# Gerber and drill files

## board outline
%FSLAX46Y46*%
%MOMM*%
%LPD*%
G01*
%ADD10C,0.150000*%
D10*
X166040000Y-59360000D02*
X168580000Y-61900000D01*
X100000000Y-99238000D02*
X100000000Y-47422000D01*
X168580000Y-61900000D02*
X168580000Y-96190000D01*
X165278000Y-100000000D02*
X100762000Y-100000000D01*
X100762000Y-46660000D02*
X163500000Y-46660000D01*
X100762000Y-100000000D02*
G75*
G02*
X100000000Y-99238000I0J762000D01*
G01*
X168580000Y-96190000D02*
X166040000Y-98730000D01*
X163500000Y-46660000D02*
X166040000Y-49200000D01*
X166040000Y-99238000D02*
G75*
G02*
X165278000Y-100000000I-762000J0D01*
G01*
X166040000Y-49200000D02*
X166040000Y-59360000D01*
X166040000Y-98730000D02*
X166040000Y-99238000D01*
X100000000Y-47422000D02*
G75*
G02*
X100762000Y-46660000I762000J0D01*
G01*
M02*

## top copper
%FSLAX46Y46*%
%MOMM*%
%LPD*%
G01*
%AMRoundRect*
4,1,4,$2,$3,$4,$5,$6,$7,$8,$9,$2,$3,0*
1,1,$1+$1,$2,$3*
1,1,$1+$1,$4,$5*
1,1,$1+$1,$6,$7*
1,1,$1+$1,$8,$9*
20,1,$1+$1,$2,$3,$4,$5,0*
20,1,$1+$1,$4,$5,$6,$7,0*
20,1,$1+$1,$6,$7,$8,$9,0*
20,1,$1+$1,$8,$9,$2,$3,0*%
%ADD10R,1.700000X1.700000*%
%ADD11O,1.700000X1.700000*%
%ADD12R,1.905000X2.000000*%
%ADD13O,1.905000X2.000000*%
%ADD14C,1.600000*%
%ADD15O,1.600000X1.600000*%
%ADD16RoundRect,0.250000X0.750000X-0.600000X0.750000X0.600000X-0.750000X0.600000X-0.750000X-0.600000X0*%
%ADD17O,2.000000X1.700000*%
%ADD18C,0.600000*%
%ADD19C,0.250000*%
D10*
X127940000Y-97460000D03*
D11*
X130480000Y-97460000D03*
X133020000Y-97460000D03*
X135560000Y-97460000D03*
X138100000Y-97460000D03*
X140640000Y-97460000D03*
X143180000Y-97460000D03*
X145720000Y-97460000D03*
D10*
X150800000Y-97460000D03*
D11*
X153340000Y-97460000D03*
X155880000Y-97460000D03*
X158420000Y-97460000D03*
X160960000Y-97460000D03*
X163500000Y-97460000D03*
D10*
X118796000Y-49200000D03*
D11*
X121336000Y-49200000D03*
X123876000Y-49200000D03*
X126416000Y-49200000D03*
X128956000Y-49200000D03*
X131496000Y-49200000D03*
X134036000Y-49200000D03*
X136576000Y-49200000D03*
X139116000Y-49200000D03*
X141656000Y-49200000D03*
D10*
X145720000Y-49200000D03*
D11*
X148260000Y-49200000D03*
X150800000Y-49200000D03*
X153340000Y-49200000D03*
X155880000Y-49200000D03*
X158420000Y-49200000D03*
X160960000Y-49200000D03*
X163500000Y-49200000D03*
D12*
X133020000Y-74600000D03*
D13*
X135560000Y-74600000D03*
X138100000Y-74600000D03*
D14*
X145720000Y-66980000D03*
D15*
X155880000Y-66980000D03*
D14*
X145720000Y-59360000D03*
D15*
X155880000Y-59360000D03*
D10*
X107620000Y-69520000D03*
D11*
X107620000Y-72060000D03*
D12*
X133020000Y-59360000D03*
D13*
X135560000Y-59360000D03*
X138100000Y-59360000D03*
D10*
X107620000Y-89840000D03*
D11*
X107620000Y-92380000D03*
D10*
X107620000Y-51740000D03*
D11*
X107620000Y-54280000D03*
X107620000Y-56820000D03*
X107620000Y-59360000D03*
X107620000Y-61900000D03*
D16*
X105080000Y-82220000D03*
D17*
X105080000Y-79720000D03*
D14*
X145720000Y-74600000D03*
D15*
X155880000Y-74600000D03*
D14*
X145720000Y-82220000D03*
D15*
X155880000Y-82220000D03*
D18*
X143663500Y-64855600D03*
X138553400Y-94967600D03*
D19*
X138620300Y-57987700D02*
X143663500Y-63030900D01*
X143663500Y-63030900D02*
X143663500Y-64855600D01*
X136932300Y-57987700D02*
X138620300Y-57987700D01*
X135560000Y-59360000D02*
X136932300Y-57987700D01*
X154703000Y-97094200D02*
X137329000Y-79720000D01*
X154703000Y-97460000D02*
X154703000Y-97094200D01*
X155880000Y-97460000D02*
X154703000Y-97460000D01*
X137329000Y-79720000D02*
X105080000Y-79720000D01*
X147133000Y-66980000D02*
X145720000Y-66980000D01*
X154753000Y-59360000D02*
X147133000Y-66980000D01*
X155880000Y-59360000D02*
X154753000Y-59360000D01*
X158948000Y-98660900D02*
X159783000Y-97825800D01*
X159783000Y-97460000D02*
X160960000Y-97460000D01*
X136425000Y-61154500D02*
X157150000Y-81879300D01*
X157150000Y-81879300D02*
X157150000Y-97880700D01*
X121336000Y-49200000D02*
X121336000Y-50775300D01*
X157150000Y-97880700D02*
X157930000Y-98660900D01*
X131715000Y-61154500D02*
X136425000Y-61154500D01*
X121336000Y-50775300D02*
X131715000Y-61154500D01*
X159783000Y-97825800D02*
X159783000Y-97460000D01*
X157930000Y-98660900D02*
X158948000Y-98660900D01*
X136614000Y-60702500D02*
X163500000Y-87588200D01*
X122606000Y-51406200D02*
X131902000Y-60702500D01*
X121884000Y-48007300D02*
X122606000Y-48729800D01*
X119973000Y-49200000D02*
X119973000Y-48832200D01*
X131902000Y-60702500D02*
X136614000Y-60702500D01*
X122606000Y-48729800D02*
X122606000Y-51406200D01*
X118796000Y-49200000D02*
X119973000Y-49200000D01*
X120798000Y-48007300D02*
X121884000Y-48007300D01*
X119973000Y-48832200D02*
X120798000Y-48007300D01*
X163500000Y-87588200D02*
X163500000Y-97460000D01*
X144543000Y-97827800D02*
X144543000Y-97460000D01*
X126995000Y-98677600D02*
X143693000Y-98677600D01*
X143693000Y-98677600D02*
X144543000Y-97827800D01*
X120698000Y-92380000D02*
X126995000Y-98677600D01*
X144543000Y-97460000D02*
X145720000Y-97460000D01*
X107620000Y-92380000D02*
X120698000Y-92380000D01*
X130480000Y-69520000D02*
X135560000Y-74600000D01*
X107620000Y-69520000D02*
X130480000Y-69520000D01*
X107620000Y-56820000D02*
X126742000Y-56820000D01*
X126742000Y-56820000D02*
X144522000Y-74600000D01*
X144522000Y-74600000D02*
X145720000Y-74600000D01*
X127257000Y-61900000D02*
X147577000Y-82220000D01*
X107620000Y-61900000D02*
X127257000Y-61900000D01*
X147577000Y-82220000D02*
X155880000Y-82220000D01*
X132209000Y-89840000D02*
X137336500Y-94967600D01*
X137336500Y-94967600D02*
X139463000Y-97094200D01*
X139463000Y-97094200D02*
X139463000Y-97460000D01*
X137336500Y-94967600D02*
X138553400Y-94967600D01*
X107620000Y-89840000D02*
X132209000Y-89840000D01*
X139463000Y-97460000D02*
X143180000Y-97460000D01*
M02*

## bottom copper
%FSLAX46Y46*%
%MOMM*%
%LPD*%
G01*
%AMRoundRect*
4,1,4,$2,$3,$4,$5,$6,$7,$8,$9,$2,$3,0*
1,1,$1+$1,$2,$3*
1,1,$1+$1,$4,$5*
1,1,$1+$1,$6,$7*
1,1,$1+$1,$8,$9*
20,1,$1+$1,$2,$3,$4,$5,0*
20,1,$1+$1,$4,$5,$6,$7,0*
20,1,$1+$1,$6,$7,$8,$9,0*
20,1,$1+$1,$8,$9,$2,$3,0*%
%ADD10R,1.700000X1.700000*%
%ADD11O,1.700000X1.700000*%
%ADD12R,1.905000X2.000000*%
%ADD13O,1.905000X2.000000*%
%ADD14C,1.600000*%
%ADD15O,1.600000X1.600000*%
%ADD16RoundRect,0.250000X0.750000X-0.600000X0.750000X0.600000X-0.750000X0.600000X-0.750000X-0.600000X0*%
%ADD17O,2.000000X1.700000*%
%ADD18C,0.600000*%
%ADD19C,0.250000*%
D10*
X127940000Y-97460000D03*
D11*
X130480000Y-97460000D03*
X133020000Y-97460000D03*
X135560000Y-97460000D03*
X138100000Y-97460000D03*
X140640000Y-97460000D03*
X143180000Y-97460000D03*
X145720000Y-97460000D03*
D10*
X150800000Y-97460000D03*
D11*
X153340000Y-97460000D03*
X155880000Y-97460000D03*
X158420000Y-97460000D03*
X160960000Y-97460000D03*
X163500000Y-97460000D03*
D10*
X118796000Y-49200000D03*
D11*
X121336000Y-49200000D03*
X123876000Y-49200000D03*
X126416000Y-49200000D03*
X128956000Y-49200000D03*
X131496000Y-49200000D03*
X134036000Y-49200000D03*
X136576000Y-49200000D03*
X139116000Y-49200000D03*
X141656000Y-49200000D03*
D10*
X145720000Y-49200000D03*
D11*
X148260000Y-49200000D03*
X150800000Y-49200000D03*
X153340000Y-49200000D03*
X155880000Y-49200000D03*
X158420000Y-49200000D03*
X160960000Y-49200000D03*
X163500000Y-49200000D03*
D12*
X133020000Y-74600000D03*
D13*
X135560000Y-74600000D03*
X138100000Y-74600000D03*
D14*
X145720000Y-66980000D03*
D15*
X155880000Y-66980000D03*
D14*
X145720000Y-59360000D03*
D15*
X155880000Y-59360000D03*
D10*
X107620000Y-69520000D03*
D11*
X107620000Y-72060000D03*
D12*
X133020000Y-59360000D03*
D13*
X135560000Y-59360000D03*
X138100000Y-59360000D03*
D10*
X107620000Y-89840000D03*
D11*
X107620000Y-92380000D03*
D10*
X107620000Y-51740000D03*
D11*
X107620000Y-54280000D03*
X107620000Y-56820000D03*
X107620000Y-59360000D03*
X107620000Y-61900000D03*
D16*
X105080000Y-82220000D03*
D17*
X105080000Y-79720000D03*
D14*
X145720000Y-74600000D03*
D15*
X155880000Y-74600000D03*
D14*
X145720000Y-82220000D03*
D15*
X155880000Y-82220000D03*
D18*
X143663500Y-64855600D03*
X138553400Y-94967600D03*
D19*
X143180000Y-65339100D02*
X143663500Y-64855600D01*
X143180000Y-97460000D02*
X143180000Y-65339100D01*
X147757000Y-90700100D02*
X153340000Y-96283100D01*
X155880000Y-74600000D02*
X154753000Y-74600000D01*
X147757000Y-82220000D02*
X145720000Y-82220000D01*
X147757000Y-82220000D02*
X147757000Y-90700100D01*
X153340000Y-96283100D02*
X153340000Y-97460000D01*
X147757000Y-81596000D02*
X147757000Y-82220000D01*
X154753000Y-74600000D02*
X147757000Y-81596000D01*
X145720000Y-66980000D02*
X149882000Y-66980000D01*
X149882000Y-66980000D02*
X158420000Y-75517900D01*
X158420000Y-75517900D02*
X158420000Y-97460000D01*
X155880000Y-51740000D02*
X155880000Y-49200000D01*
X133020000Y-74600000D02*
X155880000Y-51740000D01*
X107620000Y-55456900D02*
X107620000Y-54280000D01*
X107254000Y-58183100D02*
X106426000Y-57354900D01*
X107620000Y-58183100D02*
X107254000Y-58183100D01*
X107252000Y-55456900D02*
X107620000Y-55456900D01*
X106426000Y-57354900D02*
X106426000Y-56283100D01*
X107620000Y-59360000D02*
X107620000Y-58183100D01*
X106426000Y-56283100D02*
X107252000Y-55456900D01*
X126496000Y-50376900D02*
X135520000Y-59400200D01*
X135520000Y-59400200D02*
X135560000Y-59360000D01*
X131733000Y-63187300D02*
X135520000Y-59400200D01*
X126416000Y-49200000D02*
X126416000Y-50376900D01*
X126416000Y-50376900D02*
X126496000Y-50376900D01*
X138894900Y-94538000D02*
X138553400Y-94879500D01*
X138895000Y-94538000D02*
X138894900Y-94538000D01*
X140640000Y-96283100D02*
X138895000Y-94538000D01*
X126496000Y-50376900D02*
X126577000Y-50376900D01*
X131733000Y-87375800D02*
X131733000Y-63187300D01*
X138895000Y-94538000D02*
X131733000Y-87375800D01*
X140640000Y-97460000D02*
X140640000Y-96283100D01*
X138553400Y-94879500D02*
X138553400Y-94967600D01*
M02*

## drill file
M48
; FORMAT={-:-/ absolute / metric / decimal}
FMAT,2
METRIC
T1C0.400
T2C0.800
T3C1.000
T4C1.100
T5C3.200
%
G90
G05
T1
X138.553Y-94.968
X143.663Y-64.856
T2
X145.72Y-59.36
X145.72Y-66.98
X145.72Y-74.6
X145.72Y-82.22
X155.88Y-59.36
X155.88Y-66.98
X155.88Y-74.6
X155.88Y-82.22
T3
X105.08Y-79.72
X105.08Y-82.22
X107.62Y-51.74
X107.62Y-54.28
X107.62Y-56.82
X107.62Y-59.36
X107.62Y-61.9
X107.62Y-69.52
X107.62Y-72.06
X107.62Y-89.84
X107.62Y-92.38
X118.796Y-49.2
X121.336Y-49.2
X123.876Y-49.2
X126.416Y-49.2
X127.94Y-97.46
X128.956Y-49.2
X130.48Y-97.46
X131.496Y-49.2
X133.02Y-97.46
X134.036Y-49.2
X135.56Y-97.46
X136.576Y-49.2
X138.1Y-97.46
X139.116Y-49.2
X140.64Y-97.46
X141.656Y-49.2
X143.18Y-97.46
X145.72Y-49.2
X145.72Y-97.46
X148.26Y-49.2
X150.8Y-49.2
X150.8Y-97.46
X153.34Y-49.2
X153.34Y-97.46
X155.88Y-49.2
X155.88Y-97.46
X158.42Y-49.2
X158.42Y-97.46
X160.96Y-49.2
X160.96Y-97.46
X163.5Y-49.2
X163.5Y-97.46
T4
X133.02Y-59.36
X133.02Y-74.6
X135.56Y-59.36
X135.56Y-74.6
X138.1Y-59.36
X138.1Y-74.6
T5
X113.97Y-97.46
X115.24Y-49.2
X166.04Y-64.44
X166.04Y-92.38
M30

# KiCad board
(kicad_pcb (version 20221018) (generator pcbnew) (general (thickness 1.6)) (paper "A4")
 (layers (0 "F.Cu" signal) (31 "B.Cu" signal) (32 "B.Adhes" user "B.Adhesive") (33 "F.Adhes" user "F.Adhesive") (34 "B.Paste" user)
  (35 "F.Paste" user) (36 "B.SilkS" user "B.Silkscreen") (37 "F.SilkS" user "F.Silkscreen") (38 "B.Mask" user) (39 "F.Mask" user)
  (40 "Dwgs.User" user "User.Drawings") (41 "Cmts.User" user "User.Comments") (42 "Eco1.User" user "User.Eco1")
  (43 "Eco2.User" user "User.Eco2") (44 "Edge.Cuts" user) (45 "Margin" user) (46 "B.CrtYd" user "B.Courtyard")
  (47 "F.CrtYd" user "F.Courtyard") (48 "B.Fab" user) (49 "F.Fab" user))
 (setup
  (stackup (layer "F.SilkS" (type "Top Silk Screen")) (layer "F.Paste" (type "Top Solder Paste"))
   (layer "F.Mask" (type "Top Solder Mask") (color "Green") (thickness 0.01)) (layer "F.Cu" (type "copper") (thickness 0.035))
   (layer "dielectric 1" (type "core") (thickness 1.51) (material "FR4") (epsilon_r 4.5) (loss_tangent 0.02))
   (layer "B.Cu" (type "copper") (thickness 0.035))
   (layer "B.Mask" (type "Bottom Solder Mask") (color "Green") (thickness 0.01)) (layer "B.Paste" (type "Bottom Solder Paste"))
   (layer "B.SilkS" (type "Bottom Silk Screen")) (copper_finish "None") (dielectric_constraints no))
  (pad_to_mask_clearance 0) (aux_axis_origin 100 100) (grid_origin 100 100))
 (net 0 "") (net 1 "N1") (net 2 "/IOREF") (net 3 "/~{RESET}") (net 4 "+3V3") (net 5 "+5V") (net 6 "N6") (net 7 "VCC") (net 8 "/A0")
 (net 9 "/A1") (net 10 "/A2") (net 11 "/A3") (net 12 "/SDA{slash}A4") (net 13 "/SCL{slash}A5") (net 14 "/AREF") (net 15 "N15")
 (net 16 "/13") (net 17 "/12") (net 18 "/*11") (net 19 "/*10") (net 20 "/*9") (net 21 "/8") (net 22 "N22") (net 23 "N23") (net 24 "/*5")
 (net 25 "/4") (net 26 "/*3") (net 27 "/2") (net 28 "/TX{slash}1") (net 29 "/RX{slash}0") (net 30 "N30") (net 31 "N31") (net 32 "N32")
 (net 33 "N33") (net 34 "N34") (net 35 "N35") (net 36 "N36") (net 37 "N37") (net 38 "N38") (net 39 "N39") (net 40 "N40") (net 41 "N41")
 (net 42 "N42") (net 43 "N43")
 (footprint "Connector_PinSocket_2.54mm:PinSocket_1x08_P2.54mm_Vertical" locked (layer "F.Cu") (at 127.94 97.46 90)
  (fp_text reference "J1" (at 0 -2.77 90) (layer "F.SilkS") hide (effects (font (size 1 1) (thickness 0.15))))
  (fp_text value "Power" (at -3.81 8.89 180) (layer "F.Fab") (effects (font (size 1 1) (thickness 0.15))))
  (pad "1" thru_hole rect locked (at 0 0 90) (size 1.7 1.7) (drill 1) (layers "*.Cu" "*.Mask") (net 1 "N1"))
  (pad "2" thru_hole oval locked (at 0 2.54 90) (size 1.7 1.7) (drill 1) (layers "*.Cu" "*.Mask") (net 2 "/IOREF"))
  (pad "3" thru_hole oval locked (at 0 5.08 90) (size 1.7 1.7) (drill 1) (layers "*.Cu" "*.Mask") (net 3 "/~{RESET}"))
  (pad "4" thru_hole oval locked (at 0 7.62 90) (size 1.7 1.7) (drill 1) (layers "*.Cu" "*.Mask") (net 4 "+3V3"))
  (pad "5" thru_hole oval locked (at 0 10.16 90) (size 1.7 1.7) (drill 1) (layers "*.Cu" "*.Mask") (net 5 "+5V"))
  (pad "6" thru_hole oval locked (at 0 12.7 90) (size 1.7 1.7) (drill 1) (layers "*.Cu" "*.Mask") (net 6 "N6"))
  (pad "7" thru_hole oval locked (at 0 15.24 90) (size 1.7 1.7) (drill 1) (layers "*.Cu" "*.Mask") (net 6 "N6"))
  (pad "8" thru_hole oval locked (at 0 17.78 90) (size 1.7 1.7) (drill 1) (layers "*.Cu" "*.Mask") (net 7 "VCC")))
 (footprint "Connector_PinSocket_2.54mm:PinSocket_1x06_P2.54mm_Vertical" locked (layer "F.Cu") (at 150.8 97.46 90)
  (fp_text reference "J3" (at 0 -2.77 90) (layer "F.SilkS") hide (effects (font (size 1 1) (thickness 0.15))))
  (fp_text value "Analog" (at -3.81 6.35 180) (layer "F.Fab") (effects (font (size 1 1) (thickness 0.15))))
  (pad "1" thru_hole rect locked (at 0 0 90) (size 1.7 1.7) (drill 1) (layers "*.Cu" "*.Mask") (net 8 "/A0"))
  (pad "2" thru_hole oval locked (at 0 2.54 90) (size 1.7 1.7) (drill 1) (layers "*.Cu" "*.Mask") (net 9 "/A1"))
  (pad "3" thru_hole oval locked (at 0 5.08 90) (size 1.7 1.7) (drill 1) (layers "*.Cu" "*.Mask") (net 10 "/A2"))
  (pad "4" thru_hole oval locked (at 0 7.62 90) (size 1.7 1.7) (drill 1) (layers "*.Cu" "*.Mask") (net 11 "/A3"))
  (pad "5" thru_hole oval locked (at 0 10.16 90) (size 1.7 1.7) (drill 1) (layers "*.Cu" "*.Mask") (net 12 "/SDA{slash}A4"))
  (pad "6" thru_hole oval locked (at 0 12.7 90) (size 1.7 1.7) (drill 1) (layers "*.Cu" "*.Mask") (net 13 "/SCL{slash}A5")))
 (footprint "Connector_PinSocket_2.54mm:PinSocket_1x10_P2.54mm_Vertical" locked (layer "F.Cu") (at 118.796 49.2 90)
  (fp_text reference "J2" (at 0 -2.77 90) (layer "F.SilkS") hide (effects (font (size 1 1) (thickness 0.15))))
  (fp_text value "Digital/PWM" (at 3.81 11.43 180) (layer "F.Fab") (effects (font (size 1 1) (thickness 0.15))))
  (pad "1" thru_hole rect locked (at 0 0 90) (size 1.7 1.7) (drill 1) (layers "*.Cu" "*.Mask") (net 13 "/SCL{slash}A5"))
  (pad "2" thru_hole oval locked (at 0 2.54 90) (size 1.7 1.7) (drill 1) (layers "*.Cu" "*.Mask") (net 12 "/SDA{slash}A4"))
  (pad "3" thru_hole oval locked (at 0 5.08 90) (size 1.7 1.7) (drill 1) (layers "*.Cu" "*.Mask") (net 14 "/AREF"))
  (pad "4" thru_hole oval locked (at 0 7.62 90) (size 1.7 1.7) (drill 1) (layers "*.Cu" "*.Mask") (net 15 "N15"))
  (pad "5" thru_hole oval locked (at 0 10.16 90) (size 1.7 1.7) (drill 1) (layers "*.Cu" "*.Mask") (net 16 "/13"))
  (pad "6" thru_hole oval locked (at 0 12.7 90) (size 1.7 1.7) (drill 1) (layers "*.Cu" "*.Mask") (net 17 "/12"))
  (pad "7" thru_hole oval locked (at 0 15.24 90) (size 1.7 1.7) (drill 1) (layers "*.Cu" "*.Mask") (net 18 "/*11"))
  (pad "8" thru_hole oval locked (at 0 17.78 90) (size 1.7 1.7) (drill 1) (layers "*.Cu" "*.Mask") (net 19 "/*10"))
  (pad "9" thru_hole oval locked (at 0 20.32 90) (size 1.7 1.7) (drill 1) (layers "*.Cu" "*.Mask") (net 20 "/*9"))
  (pad "10" thru_hole oval locked (at 0 22.86 90) (size 1.7 1.7) (drill 1) (layers "*.Cu" "*.Mask") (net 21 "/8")))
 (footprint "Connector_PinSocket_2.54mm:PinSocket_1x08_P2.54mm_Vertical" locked (layer "F.Cu") (at 145.72 49.2 90)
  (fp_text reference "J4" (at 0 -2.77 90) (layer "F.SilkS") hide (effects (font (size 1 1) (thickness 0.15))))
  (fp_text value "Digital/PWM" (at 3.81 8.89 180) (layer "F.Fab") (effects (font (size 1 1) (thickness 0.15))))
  (pad "1" thru_hole rect locked (at 0 0 90) (size 1.7 1.7) (drill 1) (layers "*.Cu" "*.Mask") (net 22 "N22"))
  (pad "2" thru_hole oval locked (at 0 2.54 90) (size 1.7 1.7) (drill 1) (layers "*.Cu" "*.Mask") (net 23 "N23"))
  (pad "3" thru_hole oval locked (at 0 5.08 90) (size 1.7 1.7) (drill 1) (layers "*.Cu" "*.Mask") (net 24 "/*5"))
  (pad "4" thru_hole oval locked (at 0 7.62 90) (size 1.7 1.7) (drill 1) (layers "*.Cu" "*.Mask") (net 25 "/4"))
  (pad "5" thru_hole oval locked (at 0 10.16 90) (size 1.7 1.7) (drill 1) (layers "*.Cu" "*.Mask") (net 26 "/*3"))
  (pad "6" thru_hole oval locked (at 0 12.7 90) (size 1.7 1.7) (drill 1) (layers "*.Cu" "*.Mask") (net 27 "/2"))
  (pad "7" thru_hole oval locked (at 0 15.24 90) (size 1.7 1.7) (drill 1) (layers "*.Cu" "*.Mask") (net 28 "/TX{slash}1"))
  (pad "8" thru_hole oval locked (at 0 17.78 90) (size 1.7 1.7) (drill 1) (layers "*.Cu" "*.Mask") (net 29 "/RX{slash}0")))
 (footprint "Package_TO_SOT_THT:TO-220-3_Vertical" (layer "F.Cu") (at 133.02 74.6)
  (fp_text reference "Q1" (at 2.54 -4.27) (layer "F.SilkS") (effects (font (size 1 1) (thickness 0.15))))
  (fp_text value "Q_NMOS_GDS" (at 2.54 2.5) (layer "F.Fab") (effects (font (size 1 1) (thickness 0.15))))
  (pad "1" thru_hole rect (at 0 0) (size 1.905 2) (drill 1.1) (layers "*.Cu" "*.Mask") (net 26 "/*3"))
  (pad "2" thru_hole oval (at 2.54 0) (size 1.905 2) (drill 1.1) (layers "*.Cu" "*.Mask") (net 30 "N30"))
  (pad "3" thru_hole oval (at 5.08 0) (size 1.905 2) (drill 1.1) (layers "*.Cu" "*.Mask") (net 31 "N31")))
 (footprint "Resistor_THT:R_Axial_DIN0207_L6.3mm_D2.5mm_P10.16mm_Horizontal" (layer "F.Cu") (at 145.72 66.98)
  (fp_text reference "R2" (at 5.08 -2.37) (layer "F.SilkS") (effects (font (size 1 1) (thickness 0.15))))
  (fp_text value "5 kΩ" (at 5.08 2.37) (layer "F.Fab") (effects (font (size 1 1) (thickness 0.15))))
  (pad "1" thru_hole circle (at 0 0) (size 1.6 1.6) (drill 0.8) (layers "*.Cu" "*.Mask") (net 11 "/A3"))
  (pad "2" thru_hole oval (at 10.16 0) (size 1.6 1.6) (drill 0.8) (layers "*.Cu" "*.Mask") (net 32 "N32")))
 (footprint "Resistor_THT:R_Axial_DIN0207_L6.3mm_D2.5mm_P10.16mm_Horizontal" (layer "F.Cu") (at 145.72 59.36)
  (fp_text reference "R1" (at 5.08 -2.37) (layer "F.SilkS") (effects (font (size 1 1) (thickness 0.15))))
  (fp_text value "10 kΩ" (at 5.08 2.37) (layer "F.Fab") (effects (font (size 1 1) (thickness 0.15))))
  (pad "1" thru_hole circle (at 0 0) (size 1.6 1.6) (drill 0.8) (layers "*.Cu" "*.Mask") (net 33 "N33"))
  (pad "2" thru_hole oval (at 10.16 0) (size 1.6 1.6) (drill 0.8) (layers "*.Cu" "*.Mask") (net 11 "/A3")))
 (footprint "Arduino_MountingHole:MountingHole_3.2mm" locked (layer "F.Cu") (at 115.24 49.2)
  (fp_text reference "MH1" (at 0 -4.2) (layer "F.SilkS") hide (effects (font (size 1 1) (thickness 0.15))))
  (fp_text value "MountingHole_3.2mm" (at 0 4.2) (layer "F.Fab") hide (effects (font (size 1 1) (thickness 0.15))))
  (pad "" np_thru_hole circle locked (at 0 0) (size 3.2 3.2) (drill 3.2) (layers "*.Cu" "*.Mask")))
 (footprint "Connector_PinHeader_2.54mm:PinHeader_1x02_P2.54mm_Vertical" (layer "F.Cu") (at 107.62 69.52)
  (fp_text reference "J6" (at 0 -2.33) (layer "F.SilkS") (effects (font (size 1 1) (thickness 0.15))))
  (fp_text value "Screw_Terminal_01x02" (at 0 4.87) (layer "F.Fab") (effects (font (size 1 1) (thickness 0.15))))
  (pad "1" thru_hole rect (at 0 0) (size 1.7 1.7) (drill 1) (layers "*.Cu" "*.Mask") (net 30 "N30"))
  (pad "2" thru_hole oval (at 0 2.54) (size 1.7 1.7) (drill 1) (layers "*.Cu" "*.Mask") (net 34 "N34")))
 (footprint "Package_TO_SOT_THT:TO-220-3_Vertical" (layer "F.Cu") (at 133.02 59.36)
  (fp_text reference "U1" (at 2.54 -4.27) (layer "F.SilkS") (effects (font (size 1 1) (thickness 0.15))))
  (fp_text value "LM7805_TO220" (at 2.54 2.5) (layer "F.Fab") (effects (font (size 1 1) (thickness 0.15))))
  (pad "1" thru_hole rect (at 0 0) (size 1.905 2) (drill 1.1) (layers "*.Cu" "*.Mask") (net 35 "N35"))
  (pad "2" thru_hole oval (at 2.54 0) (size 1.905 2) (drill 1.1) (layers "*.Cu" "*.Mask") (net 6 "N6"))
  (pad "3" thru_hole oval (at 5.08 0) (size 1.905 2) (drill 1.1) (layers "*.Cu" "*.Mask") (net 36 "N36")))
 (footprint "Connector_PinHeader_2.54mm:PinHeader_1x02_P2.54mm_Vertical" (layer "F.Cu") (at 107.62 89.84)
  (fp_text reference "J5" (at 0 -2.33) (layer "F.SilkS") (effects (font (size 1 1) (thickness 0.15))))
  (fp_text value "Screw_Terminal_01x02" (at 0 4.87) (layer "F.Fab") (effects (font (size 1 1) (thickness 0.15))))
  (pad "1" thru_hole rect (at 0 0) (size 1.7 1.7) (drill 1) (layers "*.Cu" "*.Mask") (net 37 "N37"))
  (pad "2" thru_hole oval (at 0 2.54) (size 1.7 1.7) (drill 1) (layers "*.Cu" "*.Mask") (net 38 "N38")))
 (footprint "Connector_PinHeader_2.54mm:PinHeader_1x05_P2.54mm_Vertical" (layer "F.Cu") (at 107.62 51.74)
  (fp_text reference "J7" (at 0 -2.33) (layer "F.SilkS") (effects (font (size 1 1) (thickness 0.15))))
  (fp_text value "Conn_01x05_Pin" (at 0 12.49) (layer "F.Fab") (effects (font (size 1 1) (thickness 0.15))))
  (pad "1" thru_hole rect (at 0 0) (size 1.7 1.7) (drill 1) (layers "*.Cu" "*.Mask") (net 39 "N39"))
  (pad "2" thru_hole oval (at 0 2.54) (size 1.7 1.7) (drill 1) (layers "*.Cu" "*.Mask") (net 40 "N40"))
  (pad "3" thru_hole oval (at 0 5.08) (size 1.7 1.7) (drill 1) (layers "*.Cu" "*.Mask") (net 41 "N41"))
  (pad "4" thru_hole oval (at 0 7.62) (size 1.7 1.7) (drill 1) (layers "*.Cu" "*.Mask") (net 40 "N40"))
  (pad "5" thru_hole oval (at 0 10.16) (size 1.7 1.7) (drill 1) (layers "*.Cu" "*.Mask") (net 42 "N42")))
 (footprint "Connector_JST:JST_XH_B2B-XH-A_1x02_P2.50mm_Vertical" (layer "F.Cu") (at 105.08 82.22 90)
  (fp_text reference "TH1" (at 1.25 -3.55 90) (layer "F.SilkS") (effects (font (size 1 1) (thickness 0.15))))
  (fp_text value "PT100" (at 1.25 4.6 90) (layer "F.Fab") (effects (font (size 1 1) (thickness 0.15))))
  (pad "1" thru_hole roundrect (at 0 0 90) (size 1.7 2) (drill 1) (layers "*.Cu" "*.Mask") (roundrect_rratio 0.147059) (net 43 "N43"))
  (pad "2" thru_hole oval (at 2.5 0 90) (size 1.7 2) (drill 1) (layers "*.Cu" "*.Mask") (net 10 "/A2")))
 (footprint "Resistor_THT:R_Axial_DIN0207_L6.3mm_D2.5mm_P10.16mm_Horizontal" (layer "F.Cu") (at 145.72 74.6)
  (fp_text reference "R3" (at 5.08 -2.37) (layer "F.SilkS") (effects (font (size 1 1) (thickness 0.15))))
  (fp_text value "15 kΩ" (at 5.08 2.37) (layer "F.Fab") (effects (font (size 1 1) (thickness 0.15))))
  (pad "1" thru_hole circle (at 0 0) (size 1.6 1.6) (drill 0.8) (layers "*.Cu" "*.Mask") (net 41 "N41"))
  (pad "2" thru_hole oval (at 10.16 0) (size 1.6 1.6) (drill 0.8) (layers "*.Cu" "*.Mask") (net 9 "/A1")))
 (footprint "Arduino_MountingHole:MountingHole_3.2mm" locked (layer "F.Cu") (at 113.97 97.46)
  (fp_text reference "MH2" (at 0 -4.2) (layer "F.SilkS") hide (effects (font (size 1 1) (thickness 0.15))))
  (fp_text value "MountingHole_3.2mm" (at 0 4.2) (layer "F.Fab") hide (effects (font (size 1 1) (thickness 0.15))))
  (pad "" np_thru_hole circle locked (at 0 0) (size 3.2 3.2) (drill 3.2) (layers "*.Cu" "*.Mask")))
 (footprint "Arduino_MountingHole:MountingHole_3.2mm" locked (layer "F.Cu") (at 166.04 64.44)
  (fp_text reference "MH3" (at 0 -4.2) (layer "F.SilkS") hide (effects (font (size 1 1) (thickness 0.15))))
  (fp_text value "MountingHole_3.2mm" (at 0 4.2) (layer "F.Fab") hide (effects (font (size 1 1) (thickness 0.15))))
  (pad "" np_thru_hole circle locked (at 0 0) (size 3.2 3.2) (drill 3.2) (layers "*.Cu" "*.Mask")))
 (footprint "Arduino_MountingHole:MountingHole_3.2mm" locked (layer "F.Cu") (at 166.04 92.38)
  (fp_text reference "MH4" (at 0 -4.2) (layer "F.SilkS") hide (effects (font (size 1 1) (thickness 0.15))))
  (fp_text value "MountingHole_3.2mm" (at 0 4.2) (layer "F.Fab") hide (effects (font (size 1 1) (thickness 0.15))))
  (pad "" np_thru_hole circle locked (at 0 0) (size 3.2 3.2) (drill 3.2) (layers "*.Cu" "*.Mask")))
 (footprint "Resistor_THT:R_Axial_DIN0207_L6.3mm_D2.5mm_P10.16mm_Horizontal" (layer "F.Cu") (at 145.72 82.22)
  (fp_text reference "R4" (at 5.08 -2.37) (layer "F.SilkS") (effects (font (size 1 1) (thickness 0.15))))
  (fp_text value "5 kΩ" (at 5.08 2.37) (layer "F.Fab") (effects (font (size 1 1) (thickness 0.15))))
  (pad "1" thru_hole circle (at 0 0) (size 1.6 1.6) (drill 0.8) (layers "*.Cu" "*.Mask") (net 9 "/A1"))
  (pad "2" thru_hole oval (at 10.16 0) (size 1.6 1.6) (drill 0.8) (layers "*.Cu" "*.Mask") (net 42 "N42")))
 (gr_line (start 166.04 59.36) (end 168.58 61.9) (stroke (width 0.15) (type solid)) (layer "Edge.Cuts"))
 (gr_line (start 100 99.238) (end 100 47.422) (stroke (width 0.15) (type solid)) (layer "Edge.Cuts"))
 (gr_line (start 168.58 61.9) (end 168.58 96.19) (stroke (width 0.15) (type solid)) (layer "Edge.Cuts"))
 (gr_line (start 165.278 100) (end 100.762 100) (stroke (width 0.15) (type solid)) (layer "Edge.Cuts"))
 (gr_line (start 100.762 46.66) (end 163.5 46.66) (stroke (width 0.15) (type solid)) (layer "Edge.Cuts"))
 (gr_arc (start 100.762 100) (mid 100.223185 99.776815) (end 100 99.238) (stroke (width 0.15) (type solid)) (layer "Edge.Cuts"))
 (gr_line (start 168.58 96.19) (end 166.04 98.73) (stroke (width 0.15) (type solid)) (layer "Edge.Cuts"))
 (gr_line (start 163.5 46.66) (end 166.04 49.2) (stroke (width 0.15) (type solid)) (layer "Edge.Cuts"))
 (gr_arc (start 166.04 99.238) (mid 165.816815 99.776815) (end 165.278 100) (stroke (width 0.15) (type solid)) (layer "Edge.Cuts"))
 (gr_line (start 166.04 49.2) (end 166.04 59.36) (stroke (width 0.15) (type solid)) (layer "Edge.Cuts"))
 (gr_line (start 166.04 98.73) (end 166.04 99.238) (stroke (width 0.15) (type solid)) (layer "Edge.Cuts"))
 (gr_arc (start 100 47.422) (mid 100.223185 46.883185) (end 100.762 46.66) (stroke (width 0.15) (type solid)) (layer "Edge.Cuts"))
 (segment (start 138.6203 57.9877) (end 143.6635 63.0309) (width 0.25) (layer "F.Cu") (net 6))
 (segment (start 143.6635 63.0309) (end 143.6635 64.8556) (width 0.25) (layer "F.Cu") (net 6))
 (segment (start 136.9323 57.9877) (end 138.6203 57.9877) (width 0.25) (layer "F.Cu") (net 6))
 (segment (start 135.56 59.36) (end 136.9323 57.9877) (width 0.25) (layer "F.Cu") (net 6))
 (via (at 143.6635 64.8556) (size 0.6) (drill 0.4) (layers "F.Cu" "B.Cu") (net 6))
 (segment (start 143.18 65.3391) (end 143.6635 64.8556) (width 0.25) (layer "B.Cu") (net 6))
 (segment (start 143.18 97.46) (end 143.18 65.3391) (width 0.25) (layer "B.Cu") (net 6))
 (segment (start 147.757 90.7001) (end 153.34 96.2831) (width 0.25) (layer "B.Cu") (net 9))
 (segment (start 155.88 74.6) (end 154.753 74.6) (width 0.25) (layer "B.Cu") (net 9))
 (segment (start 147.757 82.22) (end 145.72 82.22) (width 0.25) (layer "B.Cu") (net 9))
 (segment (start 147.757 82.22) (end 147.757 90.7001) (width 0.25) (layer "B.Cu") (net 9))
 (segment (start 153.34 96.2831) (end 153.34 97.46) (width 0.25) (layer "B.Cu") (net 9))
 (segment (start 147.757 81.596) (end 147.757 82.22) (width 0.25) (layer "B.Cu") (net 9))
 (segment (start 154.753 74.6) (end 147.757 81.596) (width 0.25) (layer "B.Cu") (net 9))
 (segment (start 154.703 97.0942) (end 137.329 79.72) (width 0.25) (layer "F.Cu") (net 10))
 (segment (start 154.703 97.46) (end 154.703 97.0942) (width 0.25) (layer "F.Cu") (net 10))
 (segment (start 155.88 97.46) (end 154.703 97.46) (width 0.25) (layer "F.Cu") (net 10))
 (segment (start 137.329 79.72) (end 105.08 79.72) (width 0.25) (layer "F.Cu") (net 10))
 (segment (start 147.133 66.98) (end 145.72 66.98) (width 0.25) (layer "F.Cu") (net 11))
 (segment (start 154.753 59.36) (end 147.133 66.98) (width 0.25) (layer "F.Cu") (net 11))
 (segment (start 155.88 59.36) (end 154.753 59.36) (width 0.25) (layer "F.Cu") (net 11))
 (segment (start 145.72 66.98) (end 149.882 66.98) (width 0.25) (layer "B.Cu") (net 11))
 (segment (start 149.882 66.98) (end 158.42 75.5179) (width 0.25) (layer "B.Cu") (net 11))
 (segment (start 158.42 75.5179) (end 158.42 97.46) (width 0.25) (layer "B.Cu") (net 11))
 (segment (start 158.948 98.6609) (end 159.783 97.8258) (width 0.25) (layer "F.Cu") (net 12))
 (segment (start 159.783 97.46) (end 160.96 97.46) (width 0.25) (layer "F.Cu") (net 12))
 (segment (start 136.425 61.1545) (end 157.15 81.8793) (width 0.25) (layer "F.Cu") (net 12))
 (segment (start 157.15 81.8793) (end 157.15 97.8807) (width 0.25) (layer "F.Cu") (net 12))
 (segment (start 121.336 49.2) (end 121.336 50.7753) (width 0.25) (layer "F.Cu") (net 12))
 (segment (start 157.15 97.8807) (end 157.93 98.6609) (width 0.25) (layer "F.Cu") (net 12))
 (segment (start 131.715 61.1545) (end 136.425 61.1545) (width 0.25) (layer "F.Cu") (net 12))
 (segment (start 121.336 50.7753) (end 131.715 61.1545) (width 0.25) (layer "F.Cu") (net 12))
 (segment (start 159.783 97.8258) (end 159.783 97.46) (width 0.25) (layer "F.Cu") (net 12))
 (segment (start 157.93 98.6609) (end 158.948 98.6609) (width 0.25) (layer "F.Cu") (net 12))
 (segment (start 136.614 60.7025) (end 163.5 87.5882) (width 0.25) (layer "F.Cu") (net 13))
 (segment (start 122.606 51.4062) (end 131.902 60.7025) (width 0.25) (layer "F.Cu") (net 13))
 (segment (start 121.884 48.0073) (end 122.606 48.7298) (width 0.25) (layer "F.Cu") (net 13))
 (segment (start 119.973 49.2) (end 119.973 48.8322) (width 0.25) (layer "F.Cu") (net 13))
 (segment (start 131.902 60.7025) (end 136.614 60.7025) (width 0.25) (layer "F.Cu") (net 13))
 (segment (start 122.606 48.7298) (end 122.606 51.4062) (width 0.25) (layer "F.Cu") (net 13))
 (segment (start 118.796 49.2) (end 119.973 49.2) (width 0.25) (layer "F.Cu") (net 13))
 (segment (start 120.798 48.0073) (end 121.884 48.0073) (width 0.25) (layer "F.Cu") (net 13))
 (segment (start 119.973 48.8322) (end 120.798 48.0073) (width 0.25) (layer "F.Cu") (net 13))
 (segment (start 163.5 87.5882) (end 163.5 97.46) (width 0.25) (layer "F.Cu") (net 13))
 (segment (start 155.88 51.74) (end 155.88 49.2) (width 0.25) (layer "B.Cu") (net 26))
 (segment (start 133.02 74.6) (end 155.88 51.74) (width 0.25) (layer "B.Cu") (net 26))
 (segment (start 144.543 97.8278) (end 144.543 97.46) (width 0.25) (layer "F.Cu") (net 7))
 (segment (start 126.995 98.6776) (end 143.693 98.6776) (width 0.25) (layer "F.Cu") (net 7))
 (segment (start 143.693 98.6776) (end 144.543 97.8278) (width 0.25) (layer "F.Cu") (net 7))
 (segment (start 120.698 92.38) (end 126.995 98.6776) (width 0.25) (layer "F.Cu") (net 7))
 (segment (start 144.543 97.46) (end 145.72 97.46) (width 0.25) (layer "F.Cu") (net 7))
 (segment (start 107.62 92.38) (end 120.698 92.38) (width 0.25) (layer "F.Cu") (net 7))
 (segment (start 130.48 69.52) (end 135.56 74.6) (width 0.25) (layer "F.Cu") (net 30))
 (segment (start 107.62 69.52) (end 130.48 69.52) (width 0.25) (layer "F.Cu") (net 30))
 (segment (start 107.62 55.4569) (end 107.62 54.28) (width 0.25) (layer "B.Cu") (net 40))
 (segment (start 107.254 58.1831) (end 106.426 57.3549) (width 0.25) (layer "B.Cu") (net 40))
 (segment (start 107.62 58.1831) (end 107.254 58.1831) (width 0.25) (layer "B.Cu") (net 40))
 (segment (start 107.252 55.4569) (end 107.62 55.4569) (width 0.25) (layer "B.Cu") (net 40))
 (segment (start 106.426 57.3549) (end 106.426 56.2831) (width 0.25) (layer "B.Cu") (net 40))
 (segment (start 107.62 59.36) (end 107.62 58.1831) (width 0.25) (layer "B.Cu") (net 40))
 (segment (start 106.426 56.2831) (end 107.252 55.4569) (width 0.25) (layer "B.Cu") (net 40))
 (segment (start 107.62 56.82) (end 126.742 56.82) (width 0.25) (layer "F.Cu") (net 41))
 (segment (start 126.742 56.82) (end 144.522 74.6) (width 0.25) (layer "F.Cu") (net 41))
 (segment (start 144.522 74.6) (end 145.72 74.6) (width 0.25) (layer "F.Cu") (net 41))
 (segment (start 127.257 61.9) (end 147.577 82.22) (width 0.25) (layer "F.Cu") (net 42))
 (segment (start 107.62 61.9) (end 127.257 61.9) (width 0.25) (layer "F.Cu") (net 42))
 (segment (start 147.577 82.22) (end 155.88 82.22) (width 0.25) (layer "F.Cu") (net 42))
 (segment (start 132.209 89.84) (end 137.3365 94.9676) (width 0.25) (layer "F.Cu") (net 37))
 (segment (start 137.3365 94.9676) (end 139.463 97.0942) (width 0.25) (layer "F.Cu") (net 37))
 (segment (start 139.463 97.0942) (end 139.463 97.46) (width 0.25) (layer "F.Cu") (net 37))
 (segment (start 137.3365 94.9676) (end 138.5534 94.9676) (width 0.25) (layer "F.Cu") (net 37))
 (segment (start 107.62 89.84) (end 132.209 89.84) (width 0.25) (layer "F.Cu") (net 37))
 (segment (start 139.463 97.46) (end 143.18 97.46) (width 0.25) (layer "F.Cu") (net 37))
 (via (at 138.5534 94.9676) (size 0.6) (drill 0.4) (layers "F.Cu" "B.Cu") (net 37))
 (segment (start 126.496 50.3769) (end 135.52 59.4002) (width 0.25) (layer "B.Cu") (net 37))
 (segment (start 135.52 59.4002) (end 135.56 59.36) (width 0.25) (layer "B.Cu") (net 37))
 (segment (start 131.733 63.1873) (end 135.52 59.4002) (width 0.25) (layer "B.Cu") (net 37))
 (segment (start 126.416 49.2) (end 126.416 50.3769) (width 0.25) (layer "B.Cu") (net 37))
 (segment (start 126.416 50.3769) (end 126.496 50.3769) (width 0.25) (layer "B.Cu") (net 37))
 (segment (start 138.8949 94.538) (end 138.5534 94.8795) (width 0.25) (layer "B.Cu") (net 37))
 (segment (start 138.895 94.538) (end 138.8949 94.538) (width 0.25) (layer "B.Cu") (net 37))
 (segment (start 140.64 96.2831) (end 138.895 94.538) (width 0.25) (layer "B.Cu") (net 37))
 (segment (start 126.496 50.3769) (end 126.577 50.3769) (width 0.25) (layer "B.Cu") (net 37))
 (segment (start 131.733 87.3758) (end 131.733 63.1873) (width 0.25) (layer "B.Cu") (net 37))
 (segment (start 138.895 94.538) (end 131.733 87.3758) (width 0.25) (layer "B.Cu") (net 37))
 (segment (start 140.64 97.46) (end 140.64 96.2831) (width 0.25) (layer "B.Cu") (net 37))
 (segment (start 138.5534 94.8795) (end 138.5534 94.9676) (width 0.25) (layer "B.Cu") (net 37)))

